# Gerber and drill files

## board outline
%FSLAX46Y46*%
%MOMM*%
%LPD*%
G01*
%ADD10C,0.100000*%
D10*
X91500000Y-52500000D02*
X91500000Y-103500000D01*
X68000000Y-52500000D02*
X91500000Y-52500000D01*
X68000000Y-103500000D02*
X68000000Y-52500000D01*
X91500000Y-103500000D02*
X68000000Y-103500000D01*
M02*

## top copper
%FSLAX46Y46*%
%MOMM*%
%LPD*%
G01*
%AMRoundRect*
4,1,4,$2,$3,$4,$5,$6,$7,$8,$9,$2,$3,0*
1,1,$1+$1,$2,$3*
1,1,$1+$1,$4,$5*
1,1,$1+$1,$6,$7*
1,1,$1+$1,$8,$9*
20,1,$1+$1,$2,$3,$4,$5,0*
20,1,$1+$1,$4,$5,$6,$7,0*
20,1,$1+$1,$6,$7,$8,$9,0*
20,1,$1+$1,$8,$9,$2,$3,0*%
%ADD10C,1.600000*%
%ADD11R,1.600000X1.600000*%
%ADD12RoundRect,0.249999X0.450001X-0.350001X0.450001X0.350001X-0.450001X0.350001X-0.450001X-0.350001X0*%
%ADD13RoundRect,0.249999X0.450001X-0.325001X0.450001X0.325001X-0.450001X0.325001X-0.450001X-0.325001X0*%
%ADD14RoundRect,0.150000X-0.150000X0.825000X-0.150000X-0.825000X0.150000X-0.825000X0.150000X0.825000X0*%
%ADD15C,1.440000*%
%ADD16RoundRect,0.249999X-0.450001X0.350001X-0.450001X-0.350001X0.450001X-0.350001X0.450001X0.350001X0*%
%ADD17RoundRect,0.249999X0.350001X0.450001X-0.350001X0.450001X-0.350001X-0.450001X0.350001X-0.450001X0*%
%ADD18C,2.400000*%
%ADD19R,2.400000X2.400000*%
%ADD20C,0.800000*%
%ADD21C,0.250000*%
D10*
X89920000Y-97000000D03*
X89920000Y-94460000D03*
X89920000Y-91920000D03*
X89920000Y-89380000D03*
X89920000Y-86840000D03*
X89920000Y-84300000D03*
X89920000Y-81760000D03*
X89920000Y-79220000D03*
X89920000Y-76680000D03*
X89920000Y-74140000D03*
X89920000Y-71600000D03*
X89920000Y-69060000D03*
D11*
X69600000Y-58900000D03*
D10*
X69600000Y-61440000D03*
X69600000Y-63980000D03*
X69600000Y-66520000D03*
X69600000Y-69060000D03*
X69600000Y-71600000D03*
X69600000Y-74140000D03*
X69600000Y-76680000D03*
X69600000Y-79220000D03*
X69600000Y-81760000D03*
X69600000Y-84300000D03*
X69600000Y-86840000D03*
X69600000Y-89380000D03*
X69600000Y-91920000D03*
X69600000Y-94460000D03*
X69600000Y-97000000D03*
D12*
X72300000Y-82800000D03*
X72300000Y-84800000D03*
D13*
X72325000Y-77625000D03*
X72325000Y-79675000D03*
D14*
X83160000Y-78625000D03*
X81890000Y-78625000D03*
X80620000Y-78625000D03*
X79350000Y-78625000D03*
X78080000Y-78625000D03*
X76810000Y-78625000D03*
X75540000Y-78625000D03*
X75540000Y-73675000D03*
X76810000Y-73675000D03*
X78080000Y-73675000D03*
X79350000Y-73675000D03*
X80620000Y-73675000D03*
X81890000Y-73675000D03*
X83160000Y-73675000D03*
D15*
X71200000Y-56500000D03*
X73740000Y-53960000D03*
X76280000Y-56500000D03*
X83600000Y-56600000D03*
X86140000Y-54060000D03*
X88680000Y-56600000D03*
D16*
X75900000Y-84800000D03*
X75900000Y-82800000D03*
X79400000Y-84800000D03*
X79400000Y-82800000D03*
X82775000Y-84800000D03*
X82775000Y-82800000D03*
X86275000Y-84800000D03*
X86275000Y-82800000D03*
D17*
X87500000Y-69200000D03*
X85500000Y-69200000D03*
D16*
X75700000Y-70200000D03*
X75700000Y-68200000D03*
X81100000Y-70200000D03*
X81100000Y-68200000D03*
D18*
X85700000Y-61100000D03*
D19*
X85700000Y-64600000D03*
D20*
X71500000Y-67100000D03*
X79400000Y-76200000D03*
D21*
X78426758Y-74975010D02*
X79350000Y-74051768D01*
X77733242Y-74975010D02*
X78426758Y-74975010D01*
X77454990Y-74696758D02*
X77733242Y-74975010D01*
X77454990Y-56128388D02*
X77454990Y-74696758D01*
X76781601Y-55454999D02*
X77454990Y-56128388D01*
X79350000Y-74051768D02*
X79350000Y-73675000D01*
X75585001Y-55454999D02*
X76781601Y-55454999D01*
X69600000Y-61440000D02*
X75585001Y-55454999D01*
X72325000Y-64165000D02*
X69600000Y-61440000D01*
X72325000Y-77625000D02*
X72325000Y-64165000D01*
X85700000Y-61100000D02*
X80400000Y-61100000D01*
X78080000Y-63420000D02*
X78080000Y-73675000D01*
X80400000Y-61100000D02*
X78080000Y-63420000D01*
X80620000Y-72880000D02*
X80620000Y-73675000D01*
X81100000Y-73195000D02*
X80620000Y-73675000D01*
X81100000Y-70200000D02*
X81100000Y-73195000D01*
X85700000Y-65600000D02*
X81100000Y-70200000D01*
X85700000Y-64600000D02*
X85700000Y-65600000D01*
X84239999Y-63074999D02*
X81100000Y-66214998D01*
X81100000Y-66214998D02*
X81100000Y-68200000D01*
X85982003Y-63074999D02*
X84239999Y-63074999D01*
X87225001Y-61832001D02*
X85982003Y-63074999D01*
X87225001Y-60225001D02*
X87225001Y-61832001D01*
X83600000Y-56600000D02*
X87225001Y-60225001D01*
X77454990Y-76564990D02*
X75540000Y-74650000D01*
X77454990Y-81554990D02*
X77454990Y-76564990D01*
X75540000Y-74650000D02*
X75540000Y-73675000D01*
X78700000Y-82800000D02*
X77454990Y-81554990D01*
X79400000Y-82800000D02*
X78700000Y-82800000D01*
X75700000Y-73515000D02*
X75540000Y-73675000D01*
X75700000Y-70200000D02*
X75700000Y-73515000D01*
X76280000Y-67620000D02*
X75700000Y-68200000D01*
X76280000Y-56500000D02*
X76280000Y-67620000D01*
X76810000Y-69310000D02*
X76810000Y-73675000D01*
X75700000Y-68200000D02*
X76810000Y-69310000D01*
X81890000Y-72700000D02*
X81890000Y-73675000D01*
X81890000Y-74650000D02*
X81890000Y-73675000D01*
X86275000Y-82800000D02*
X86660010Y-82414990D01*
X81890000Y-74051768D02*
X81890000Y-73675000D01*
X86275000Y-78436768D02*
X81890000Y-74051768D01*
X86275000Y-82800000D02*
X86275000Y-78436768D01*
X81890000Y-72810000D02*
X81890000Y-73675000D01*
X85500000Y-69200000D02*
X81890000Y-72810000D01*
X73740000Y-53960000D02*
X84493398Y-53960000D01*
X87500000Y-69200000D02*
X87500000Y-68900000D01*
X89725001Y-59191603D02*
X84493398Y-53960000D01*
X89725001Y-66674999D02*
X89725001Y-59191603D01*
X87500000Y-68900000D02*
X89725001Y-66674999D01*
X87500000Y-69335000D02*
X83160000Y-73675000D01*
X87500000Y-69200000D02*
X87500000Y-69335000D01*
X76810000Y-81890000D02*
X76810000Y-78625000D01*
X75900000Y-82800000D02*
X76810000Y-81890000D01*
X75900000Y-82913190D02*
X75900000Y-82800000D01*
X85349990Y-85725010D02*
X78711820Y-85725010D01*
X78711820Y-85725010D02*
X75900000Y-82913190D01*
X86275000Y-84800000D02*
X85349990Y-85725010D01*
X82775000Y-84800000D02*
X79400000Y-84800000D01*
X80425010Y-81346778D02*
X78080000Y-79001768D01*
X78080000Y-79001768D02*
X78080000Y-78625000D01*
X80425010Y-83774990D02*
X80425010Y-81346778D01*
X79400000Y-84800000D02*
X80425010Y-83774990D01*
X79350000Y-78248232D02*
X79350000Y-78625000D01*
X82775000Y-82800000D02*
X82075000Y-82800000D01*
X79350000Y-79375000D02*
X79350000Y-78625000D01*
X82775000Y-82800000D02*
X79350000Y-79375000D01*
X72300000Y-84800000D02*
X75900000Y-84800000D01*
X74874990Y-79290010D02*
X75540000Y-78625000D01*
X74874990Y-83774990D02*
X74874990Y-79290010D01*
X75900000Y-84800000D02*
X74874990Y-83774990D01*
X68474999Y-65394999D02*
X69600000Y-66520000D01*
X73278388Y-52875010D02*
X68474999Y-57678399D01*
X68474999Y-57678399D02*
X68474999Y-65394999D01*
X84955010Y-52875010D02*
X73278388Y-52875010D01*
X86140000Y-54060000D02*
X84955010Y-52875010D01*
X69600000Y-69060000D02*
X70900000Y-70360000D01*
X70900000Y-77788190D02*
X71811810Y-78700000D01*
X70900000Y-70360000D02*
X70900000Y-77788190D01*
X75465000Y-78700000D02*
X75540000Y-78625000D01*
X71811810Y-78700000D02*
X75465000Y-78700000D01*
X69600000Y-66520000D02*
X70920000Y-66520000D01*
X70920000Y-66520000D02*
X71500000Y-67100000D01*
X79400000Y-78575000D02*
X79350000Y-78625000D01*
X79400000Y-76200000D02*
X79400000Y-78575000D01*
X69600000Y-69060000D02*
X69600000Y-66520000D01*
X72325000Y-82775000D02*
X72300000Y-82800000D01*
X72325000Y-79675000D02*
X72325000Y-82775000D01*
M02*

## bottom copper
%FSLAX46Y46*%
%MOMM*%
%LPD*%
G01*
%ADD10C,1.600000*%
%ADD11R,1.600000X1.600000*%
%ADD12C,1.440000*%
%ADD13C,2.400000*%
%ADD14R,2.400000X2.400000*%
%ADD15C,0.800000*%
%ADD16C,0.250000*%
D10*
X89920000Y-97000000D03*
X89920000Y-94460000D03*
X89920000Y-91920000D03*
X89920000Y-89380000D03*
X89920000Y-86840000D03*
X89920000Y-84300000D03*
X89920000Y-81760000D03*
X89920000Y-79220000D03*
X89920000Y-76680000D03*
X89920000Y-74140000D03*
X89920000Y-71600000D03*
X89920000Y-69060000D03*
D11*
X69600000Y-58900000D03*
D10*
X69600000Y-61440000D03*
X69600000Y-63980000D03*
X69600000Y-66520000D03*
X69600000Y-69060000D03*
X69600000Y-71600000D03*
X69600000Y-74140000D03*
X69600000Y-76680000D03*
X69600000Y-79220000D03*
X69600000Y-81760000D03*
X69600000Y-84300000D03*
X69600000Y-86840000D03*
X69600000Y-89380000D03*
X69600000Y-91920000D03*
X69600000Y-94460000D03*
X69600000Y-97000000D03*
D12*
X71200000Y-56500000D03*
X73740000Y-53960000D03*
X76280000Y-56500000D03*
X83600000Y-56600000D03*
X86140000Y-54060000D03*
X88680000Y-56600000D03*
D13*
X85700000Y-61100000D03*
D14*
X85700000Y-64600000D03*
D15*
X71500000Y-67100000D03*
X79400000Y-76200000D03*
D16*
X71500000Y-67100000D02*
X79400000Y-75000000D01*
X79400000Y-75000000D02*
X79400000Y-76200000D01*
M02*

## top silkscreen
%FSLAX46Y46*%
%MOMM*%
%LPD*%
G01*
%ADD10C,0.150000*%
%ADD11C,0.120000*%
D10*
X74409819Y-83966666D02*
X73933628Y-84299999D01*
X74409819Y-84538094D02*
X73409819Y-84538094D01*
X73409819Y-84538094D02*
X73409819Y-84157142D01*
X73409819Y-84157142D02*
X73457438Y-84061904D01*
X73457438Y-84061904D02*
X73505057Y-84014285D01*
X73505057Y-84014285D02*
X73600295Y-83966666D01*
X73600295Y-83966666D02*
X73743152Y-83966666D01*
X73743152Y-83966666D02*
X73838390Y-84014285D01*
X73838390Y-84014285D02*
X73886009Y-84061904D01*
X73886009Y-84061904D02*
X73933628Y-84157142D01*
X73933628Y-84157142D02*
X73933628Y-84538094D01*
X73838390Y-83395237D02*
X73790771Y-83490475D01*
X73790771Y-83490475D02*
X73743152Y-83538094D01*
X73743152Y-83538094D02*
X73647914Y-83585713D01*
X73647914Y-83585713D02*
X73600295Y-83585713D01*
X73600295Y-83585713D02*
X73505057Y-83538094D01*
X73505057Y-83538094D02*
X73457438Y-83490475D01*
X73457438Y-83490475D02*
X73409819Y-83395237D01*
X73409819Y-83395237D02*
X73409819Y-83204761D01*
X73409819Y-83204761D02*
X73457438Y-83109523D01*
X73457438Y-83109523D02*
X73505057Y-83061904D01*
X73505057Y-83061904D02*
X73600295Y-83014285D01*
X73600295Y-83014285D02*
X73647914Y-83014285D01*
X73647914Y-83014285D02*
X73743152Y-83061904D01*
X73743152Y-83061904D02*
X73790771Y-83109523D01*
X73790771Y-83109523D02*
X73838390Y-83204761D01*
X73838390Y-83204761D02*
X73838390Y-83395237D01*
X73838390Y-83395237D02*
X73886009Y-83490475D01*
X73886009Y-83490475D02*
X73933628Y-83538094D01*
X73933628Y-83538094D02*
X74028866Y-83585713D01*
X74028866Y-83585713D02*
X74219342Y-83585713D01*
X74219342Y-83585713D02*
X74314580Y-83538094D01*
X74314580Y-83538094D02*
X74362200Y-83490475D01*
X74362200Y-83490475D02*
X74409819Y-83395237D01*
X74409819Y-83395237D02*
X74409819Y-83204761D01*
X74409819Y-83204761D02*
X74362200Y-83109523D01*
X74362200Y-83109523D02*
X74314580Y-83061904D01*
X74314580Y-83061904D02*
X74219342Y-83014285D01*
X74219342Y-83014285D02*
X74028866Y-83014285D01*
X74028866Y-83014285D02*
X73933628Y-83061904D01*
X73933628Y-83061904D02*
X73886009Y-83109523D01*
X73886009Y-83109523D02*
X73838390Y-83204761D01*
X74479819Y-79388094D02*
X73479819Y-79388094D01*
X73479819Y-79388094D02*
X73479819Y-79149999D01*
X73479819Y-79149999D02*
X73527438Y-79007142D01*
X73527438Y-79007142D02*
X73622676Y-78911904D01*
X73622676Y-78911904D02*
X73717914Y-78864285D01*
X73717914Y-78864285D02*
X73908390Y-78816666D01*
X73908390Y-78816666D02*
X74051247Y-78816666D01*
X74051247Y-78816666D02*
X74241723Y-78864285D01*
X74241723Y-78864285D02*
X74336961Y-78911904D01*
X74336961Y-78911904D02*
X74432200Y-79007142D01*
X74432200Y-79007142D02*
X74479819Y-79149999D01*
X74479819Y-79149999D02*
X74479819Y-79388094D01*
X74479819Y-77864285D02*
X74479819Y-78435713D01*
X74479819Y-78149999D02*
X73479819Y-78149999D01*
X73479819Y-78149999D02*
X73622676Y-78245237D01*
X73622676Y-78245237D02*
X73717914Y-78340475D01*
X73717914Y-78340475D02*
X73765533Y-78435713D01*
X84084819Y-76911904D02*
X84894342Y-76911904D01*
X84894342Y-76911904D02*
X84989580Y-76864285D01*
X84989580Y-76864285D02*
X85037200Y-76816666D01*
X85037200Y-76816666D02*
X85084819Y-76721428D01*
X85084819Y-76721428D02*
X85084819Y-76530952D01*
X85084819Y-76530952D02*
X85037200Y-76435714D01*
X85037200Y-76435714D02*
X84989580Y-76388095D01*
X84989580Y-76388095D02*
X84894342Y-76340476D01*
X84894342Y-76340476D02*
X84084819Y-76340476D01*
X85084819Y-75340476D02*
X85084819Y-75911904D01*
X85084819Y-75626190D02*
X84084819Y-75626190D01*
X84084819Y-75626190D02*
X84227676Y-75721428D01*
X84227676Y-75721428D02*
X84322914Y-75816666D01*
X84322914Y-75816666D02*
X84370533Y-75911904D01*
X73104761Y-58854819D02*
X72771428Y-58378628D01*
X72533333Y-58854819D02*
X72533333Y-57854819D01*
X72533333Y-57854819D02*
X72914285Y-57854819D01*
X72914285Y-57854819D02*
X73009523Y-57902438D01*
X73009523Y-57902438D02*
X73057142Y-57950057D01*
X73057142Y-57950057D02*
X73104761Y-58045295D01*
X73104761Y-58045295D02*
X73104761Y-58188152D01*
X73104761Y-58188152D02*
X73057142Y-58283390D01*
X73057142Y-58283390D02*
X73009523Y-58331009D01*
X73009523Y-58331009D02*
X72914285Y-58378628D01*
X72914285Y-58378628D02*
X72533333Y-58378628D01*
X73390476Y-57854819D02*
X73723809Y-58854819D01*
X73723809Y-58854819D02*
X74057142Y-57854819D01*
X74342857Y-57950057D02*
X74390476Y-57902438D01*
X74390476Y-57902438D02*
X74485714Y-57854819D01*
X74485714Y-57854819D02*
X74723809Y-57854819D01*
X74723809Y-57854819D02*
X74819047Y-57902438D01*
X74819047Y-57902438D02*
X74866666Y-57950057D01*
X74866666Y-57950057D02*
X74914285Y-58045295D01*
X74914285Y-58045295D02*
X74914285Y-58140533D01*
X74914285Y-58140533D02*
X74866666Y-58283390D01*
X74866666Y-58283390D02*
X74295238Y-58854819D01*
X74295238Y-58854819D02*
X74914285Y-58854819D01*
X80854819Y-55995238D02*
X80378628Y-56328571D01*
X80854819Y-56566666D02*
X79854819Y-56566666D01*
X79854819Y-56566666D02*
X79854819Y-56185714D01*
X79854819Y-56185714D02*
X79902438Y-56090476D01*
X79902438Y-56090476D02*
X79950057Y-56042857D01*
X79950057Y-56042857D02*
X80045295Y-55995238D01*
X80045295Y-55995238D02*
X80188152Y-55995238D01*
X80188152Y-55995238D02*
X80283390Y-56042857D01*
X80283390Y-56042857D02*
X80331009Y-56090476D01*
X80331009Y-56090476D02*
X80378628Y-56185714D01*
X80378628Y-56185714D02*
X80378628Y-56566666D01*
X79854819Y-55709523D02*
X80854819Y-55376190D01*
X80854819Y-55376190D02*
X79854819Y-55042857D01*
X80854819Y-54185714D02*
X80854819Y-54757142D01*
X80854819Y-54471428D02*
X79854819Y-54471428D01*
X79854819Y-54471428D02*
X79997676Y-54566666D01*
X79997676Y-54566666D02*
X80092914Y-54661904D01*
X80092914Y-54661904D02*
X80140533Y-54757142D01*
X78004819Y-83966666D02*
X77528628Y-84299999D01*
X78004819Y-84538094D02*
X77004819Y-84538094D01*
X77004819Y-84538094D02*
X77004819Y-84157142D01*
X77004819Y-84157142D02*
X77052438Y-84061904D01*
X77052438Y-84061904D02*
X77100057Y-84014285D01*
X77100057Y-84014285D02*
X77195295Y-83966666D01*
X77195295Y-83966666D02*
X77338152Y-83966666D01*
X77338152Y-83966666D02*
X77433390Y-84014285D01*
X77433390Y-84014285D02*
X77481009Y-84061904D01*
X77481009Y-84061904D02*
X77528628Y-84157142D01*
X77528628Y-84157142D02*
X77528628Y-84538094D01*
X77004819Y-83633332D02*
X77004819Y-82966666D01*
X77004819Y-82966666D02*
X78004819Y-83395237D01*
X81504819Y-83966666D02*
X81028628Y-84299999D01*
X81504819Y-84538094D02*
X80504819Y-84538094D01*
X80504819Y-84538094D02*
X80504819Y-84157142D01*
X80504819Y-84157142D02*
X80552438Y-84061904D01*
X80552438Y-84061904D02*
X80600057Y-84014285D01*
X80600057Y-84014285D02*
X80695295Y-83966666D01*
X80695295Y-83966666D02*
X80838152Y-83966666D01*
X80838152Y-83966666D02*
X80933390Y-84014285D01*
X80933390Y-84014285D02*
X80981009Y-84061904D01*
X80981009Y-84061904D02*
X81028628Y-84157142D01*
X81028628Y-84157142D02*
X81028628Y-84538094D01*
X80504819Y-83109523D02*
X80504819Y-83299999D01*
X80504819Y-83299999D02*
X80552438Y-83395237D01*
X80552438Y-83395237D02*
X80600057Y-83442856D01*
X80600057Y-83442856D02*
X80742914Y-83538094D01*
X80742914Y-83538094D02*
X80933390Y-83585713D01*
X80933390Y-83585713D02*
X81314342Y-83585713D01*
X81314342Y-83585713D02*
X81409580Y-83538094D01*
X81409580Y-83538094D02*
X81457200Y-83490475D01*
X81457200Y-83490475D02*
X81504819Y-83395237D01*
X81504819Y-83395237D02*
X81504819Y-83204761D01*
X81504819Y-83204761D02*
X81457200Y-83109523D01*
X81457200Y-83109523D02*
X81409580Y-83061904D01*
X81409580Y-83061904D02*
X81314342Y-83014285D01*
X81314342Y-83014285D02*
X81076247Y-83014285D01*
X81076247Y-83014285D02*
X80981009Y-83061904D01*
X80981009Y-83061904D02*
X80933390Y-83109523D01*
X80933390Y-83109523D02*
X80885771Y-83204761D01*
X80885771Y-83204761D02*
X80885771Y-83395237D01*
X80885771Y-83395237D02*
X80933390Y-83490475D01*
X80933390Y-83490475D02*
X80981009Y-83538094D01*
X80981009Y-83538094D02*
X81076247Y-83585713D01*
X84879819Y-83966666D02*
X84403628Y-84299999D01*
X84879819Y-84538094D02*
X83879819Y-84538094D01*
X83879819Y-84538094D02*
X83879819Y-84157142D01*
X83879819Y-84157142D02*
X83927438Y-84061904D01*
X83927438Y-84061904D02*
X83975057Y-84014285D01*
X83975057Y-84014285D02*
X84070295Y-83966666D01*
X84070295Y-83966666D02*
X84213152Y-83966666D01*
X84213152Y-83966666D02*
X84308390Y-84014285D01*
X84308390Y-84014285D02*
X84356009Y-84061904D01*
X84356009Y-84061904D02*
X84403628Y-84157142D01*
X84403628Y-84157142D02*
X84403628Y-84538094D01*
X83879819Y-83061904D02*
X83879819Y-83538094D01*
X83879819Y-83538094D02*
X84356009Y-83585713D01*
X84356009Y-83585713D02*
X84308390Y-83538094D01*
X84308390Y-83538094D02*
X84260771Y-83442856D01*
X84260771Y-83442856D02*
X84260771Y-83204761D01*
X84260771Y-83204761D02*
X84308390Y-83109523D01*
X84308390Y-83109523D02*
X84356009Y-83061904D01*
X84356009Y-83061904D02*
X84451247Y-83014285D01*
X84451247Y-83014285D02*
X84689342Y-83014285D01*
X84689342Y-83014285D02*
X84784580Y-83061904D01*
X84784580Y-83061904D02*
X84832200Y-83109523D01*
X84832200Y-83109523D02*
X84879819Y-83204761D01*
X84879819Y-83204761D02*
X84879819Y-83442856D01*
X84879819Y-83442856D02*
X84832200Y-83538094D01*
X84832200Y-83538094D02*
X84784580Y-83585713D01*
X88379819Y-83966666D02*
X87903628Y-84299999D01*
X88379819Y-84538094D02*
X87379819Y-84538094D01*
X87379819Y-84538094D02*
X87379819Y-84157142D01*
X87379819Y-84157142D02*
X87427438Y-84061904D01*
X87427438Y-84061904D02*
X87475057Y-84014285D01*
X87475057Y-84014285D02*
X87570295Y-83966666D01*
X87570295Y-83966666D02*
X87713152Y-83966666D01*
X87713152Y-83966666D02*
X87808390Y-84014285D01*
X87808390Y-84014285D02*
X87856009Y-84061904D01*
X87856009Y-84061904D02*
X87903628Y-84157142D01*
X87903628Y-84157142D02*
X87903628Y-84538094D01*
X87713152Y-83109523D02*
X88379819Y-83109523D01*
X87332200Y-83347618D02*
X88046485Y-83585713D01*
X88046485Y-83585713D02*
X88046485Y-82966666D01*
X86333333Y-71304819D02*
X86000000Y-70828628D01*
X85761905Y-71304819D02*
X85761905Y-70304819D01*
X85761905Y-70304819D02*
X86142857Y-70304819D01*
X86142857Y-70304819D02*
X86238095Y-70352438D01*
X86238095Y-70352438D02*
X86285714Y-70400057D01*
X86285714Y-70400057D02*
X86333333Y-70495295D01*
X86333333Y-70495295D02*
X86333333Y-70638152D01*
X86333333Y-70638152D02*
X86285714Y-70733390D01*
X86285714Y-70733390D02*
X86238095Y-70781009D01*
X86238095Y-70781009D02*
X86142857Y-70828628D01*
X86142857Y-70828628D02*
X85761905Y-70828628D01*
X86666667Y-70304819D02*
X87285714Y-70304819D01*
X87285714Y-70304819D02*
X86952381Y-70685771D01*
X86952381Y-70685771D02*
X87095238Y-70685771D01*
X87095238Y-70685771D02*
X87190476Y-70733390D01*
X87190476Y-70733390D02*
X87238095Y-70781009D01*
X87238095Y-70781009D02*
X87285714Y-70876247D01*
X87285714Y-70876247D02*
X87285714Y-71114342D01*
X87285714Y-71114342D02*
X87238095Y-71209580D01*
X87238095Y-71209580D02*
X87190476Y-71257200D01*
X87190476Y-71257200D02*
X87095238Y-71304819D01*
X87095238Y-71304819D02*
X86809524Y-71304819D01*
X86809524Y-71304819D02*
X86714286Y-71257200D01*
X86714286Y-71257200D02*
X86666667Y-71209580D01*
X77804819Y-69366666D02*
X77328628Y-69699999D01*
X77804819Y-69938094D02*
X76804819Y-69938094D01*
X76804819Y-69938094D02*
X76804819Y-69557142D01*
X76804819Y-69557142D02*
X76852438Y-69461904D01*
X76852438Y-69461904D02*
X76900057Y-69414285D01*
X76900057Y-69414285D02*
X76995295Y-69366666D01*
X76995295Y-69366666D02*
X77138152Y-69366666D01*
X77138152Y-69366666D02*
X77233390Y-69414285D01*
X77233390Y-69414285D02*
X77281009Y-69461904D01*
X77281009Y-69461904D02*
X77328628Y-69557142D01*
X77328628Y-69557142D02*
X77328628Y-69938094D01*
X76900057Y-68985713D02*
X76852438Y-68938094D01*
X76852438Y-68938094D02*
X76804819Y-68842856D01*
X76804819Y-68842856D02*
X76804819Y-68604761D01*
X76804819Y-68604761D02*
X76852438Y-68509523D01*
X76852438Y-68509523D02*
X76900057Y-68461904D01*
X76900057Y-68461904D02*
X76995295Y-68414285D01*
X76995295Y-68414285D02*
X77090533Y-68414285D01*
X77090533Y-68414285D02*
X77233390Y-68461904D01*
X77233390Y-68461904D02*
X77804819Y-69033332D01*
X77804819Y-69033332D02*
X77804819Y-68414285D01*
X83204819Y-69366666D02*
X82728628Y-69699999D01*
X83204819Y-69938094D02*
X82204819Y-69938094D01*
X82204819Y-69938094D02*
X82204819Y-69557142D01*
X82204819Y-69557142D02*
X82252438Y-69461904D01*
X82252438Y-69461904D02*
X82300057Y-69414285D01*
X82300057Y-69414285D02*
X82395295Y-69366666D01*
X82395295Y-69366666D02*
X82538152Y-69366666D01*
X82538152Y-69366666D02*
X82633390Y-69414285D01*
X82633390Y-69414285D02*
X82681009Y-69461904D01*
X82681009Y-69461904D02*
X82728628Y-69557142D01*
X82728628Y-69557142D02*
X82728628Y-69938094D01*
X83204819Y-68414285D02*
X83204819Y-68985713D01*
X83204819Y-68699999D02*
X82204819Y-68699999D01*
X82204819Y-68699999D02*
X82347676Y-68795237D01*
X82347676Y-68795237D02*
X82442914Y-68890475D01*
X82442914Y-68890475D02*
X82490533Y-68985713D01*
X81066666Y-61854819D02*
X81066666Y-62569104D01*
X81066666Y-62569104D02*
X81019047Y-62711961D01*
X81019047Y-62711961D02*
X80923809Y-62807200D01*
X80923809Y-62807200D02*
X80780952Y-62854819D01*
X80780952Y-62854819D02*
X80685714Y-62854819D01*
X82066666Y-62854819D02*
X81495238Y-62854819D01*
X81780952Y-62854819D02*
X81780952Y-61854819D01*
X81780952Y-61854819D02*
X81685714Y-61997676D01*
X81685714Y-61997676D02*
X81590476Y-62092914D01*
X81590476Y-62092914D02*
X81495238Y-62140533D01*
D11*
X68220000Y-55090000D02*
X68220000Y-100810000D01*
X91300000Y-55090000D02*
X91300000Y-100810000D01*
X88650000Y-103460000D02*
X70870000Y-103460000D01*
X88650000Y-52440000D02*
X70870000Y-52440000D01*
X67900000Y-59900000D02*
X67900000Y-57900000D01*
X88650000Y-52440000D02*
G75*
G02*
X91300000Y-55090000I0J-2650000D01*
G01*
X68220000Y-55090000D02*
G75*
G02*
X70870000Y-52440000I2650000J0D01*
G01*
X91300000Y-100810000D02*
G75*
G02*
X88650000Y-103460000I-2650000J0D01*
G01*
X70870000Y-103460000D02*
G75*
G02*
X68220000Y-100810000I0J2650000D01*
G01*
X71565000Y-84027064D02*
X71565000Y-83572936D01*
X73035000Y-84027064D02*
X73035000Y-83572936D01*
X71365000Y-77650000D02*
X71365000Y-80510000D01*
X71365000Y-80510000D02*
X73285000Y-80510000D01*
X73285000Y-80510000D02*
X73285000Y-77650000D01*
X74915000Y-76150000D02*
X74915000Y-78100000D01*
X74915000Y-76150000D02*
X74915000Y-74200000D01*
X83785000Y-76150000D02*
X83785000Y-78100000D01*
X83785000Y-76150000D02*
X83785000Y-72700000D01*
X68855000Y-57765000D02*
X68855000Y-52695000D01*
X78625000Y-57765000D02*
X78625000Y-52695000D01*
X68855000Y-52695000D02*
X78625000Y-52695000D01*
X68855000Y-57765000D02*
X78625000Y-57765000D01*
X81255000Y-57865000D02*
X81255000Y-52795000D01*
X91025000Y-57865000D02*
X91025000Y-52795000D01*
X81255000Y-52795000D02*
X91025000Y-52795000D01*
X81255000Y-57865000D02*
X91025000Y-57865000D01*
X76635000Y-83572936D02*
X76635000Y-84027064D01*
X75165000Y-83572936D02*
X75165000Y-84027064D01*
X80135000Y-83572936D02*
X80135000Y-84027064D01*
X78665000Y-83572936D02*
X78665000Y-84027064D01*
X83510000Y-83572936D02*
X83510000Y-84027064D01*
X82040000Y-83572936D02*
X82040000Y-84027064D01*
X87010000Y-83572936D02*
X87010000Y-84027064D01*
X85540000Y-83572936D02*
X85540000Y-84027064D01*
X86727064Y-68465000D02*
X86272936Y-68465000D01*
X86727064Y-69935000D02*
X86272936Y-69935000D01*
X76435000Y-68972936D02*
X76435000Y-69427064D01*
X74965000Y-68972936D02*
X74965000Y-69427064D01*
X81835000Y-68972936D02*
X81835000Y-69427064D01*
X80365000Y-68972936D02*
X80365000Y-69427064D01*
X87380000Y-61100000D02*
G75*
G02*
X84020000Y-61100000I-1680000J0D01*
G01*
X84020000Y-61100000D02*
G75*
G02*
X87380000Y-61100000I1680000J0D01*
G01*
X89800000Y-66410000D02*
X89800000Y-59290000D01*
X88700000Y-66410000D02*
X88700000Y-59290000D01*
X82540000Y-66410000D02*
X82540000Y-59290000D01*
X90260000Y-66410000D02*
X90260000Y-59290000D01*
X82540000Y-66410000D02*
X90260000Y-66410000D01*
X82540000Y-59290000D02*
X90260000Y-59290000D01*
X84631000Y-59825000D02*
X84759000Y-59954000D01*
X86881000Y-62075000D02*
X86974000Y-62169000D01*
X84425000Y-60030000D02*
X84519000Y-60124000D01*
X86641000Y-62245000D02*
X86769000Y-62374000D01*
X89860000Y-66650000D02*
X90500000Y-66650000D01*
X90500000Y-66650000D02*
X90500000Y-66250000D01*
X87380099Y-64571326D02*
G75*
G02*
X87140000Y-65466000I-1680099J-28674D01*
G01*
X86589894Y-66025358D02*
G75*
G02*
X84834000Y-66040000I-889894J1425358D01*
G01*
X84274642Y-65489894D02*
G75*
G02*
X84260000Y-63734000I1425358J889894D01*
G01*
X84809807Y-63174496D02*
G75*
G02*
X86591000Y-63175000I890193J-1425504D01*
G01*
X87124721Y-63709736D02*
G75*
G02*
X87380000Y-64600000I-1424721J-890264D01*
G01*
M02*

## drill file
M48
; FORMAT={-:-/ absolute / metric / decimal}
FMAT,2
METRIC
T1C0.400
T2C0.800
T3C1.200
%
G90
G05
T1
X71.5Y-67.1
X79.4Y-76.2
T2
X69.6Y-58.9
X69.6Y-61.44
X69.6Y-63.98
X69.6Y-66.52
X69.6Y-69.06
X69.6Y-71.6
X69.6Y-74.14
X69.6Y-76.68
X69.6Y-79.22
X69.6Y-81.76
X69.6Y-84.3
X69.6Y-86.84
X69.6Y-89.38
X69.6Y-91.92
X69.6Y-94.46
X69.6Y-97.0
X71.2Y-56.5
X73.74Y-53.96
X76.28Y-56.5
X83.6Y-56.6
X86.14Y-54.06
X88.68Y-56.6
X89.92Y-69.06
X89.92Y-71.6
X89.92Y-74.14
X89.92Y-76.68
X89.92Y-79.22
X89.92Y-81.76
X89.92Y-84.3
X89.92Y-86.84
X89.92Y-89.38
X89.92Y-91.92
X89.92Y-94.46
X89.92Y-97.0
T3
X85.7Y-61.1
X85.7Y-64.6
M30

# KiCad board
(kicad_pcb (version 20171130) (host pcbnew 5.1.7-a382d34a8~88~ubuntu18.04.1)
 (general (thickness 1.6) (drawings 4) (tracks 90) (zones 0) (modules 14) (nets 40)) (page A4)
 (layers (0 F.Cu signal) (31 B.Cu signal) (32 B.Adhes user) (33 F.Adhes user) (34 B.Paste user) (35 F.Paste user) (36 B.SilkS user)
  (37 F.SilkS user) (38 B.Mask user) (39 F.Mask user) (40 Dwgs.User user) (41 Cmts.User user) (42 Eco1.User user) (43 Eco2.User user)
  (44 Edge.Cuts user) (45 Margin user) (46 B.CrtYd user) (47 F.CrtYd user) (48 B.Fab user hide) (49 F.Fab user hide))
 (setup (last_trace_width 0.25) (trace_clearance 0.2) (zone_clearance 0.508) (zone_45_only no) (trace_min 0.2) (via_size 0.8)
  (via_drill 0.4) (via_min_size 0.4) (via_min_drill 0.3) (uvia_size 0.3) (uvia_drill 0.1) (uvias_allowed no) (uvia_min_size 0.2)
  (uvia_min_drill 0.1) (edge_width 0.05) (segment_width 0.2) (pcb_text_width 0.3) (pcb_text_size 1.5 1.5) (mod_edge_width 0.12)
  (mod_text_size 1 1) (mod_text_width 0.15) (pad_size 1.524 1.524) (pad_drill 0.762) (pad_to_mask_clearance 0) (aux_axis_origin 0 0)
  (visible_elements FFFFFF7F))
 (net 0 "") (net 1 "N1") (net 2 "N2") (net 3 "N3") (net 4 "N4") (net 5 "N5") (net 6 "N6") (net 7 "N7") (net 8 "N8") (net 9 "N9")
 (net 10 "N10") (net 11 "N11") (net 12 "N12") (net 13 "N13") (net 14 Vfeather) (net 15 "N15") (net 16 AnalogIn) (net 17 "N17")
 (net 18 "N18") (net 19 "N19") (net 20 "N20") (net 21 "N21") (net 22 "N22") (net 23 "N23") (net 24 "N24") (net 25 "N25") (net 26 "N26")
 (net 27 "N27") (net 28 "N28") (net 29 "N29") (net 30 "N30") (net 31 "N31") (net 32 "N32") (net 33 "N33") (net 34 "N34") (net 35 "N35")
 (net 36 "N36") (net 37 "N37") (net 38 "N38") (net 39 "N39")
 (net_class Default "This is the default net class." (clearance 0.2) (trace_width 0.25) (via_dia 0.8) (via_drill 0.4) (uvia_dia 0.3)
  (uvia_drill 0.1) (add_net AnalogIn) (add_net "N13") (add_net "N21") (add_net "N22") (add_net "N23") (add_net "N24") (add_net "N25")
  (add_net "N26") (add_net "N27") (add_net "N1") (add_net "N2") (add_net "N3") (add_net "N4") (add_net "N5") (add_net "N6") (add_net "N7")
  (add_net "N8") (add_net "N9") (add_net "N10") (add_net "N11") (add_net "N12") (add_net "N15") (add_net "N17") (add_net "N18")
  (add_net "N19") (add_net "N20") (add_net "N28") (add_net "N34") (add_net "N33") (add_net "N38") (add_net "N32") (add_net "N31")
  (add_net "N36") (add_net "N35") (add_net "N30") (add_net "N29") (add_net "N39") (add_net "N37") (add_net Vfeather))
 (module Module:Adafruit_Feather (layer F.Cu) (at 69.6 58.9)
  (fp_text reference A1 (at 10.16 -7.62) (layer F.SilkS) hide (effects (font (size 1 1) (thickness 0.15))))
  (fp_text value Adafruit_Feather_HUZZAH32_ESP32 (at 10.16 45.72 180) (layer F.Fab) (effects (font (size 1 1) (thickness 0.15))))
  (fp_line (start -1.38 -3.81) (end -1.38 41.91) (layer F.SilkS) (width 0.12))
  (fp_line (start 21.7 -3.81) (end 21.7 41.91) (layer F.SilkS) (width 0.12))
  (fp_line (start 19.05 44.56) (end 1.27 44.56) (layer F.SilkS) (width 0.12))
  (fp_line (start 19.05 -6.46) (end 1.27 -6.46) (layer F.SilkS) (width 0.12))
  (fp_line (start -1.7 1) (end -1.7 -1) (layer F.SilkS) (width 0.12))
  (fp_arc (start 19.05 -3.81) (end 21.7 -3.81) (angle -90) (layer F.SilkS) (width 0.12))
  (fp_arc (start 1.27 -3.81) (end 1.27 -6.46) (angle -90) (layer F.SilkS) (width 0.12))
  (fp_arc (start 19.05 41.91) (end 19.05 44.56) (angle -90) (layer F.SilkS) (width 0.12))
  (fp_arc (start 1.27 41.91) (end -1.38 41.91) (angle -90) (layer F.SilkS) (width 0.12))
  (pad 17 thru_hole circle (at 20.32 38.1 180) (size 1.6 1.6) (drill 0.8) (layers *.Cu *.Mask) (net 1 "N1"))
  (pad 18 thru_hole circle (at 20.32 35.56 180) (size 1.6 1.6) (drill 0.8) (layers *.Cu *.Mask) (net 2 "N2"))
  (pad 19 thru_hole circle (at 20.32 33.02 180) (size 1.6 1.6) (drill 0.8) (layers *.Cu *.Mask) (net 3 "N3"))
  (pad 20 thru_hole circle (at 20.32 30.48 180) (size 1.6 1.6) (drill 0.8) (layers *.Cu *.Mask) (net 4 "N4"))
  (pad 21 thru_hole circle (at 20.32 27.94 180) (size 1.6 1.6) (drill 0.8) (layers *.Cu *.Mask) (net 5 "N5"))
  (pad 22 thru_hole circle (at 20.32 25.4 180) (size 1.6 1.6) (drill 0.8) (layers *.Cu *.Mask) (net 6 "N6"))
  (pad 23 thru_hole circle (at 20.32 22.86 180) (size 1.6 1.6) (drill 0.8) (layers *.Cu *.Mask) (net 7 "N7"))
  (pad 24 thru_hole circle (at 20.32 20.32 180) (size 1.6 1.6) (drill 0.8) (layers *.Cu *.Mask) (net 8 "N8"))
  (pad 25 thru_hole circle (at 20.32 17.78 180) (size 1.6 1.6) (drill 0.8) (layers *.Cu *.Mask) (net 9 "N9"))
  (pad 26 thru_hole circle (at 20.32 15.24 180) (size 1.6 1.6) (drill 0.8) (layers *.Cu *.Mask) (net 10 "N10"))
  (pad 27 thru_hole circle (at 20.32 12.7 180) (size 1.6 1.6) (drill 0.8) (layers *.Cu *.Mask) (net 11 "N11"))
  (pad 28 thru_hole circle (at 20.32 10.16 180) (size 1.6 1.6) (drill 0.8) (layers *.Cu *.Mask) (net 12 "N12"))
  (pad 1 thru_hole rect (at 0 0 180) (size 1.6 1.6) (drill 0.8) (layers *.Cu *.Mask) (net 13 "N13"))
  (pad 2 thru_hole circle (at 0 2.54 180) (size 1.6 1.6) (drill 0.8) (layers *.Cu *.Mask) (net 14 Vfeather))
  (pad 3 thru_hole circle (at 0 5.08 180) (size 1.6 1.6) (drill 0.8) (layers *.Cu *.Mask) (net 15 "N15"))
  (pad 4 thru_hole circle (at 0 7.62 180) (size 1.6 1.6) (drill 0.8) (layers *.Cu *.Mask) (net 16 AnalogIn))
  (pad 5 thru_hole circle (at 0 10.16 180) (size 1.6 1.6) (drill 0.8) (layers *.Cu *.Mask) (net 16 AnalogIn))
  (pad 6 thru_hole circle (at 0 12.7 180) (size 1.6 1.6) (drill 0.8) (layers *.Cu *.Mask) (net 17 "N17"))
  (pad 7 thru_hole circle (at 0 15.24 180) (size 1.6 1.6) (drill 0.8) (layers *.Cu *.Mask) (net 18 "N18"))
  (pad 8 thru_hole circle (at 0 17.78 180) (size 1.6 1.6) (drill 0.8) (layers *.Cu *.Mask) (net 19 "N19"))
  (pad 9 thru_hole circle (at 0 20.32 180) (size 1.6 1.6) (drill 0.8) (layers *.Cu *.Mask) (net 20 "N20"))
  (pad 10 thru_hole circle (at 0 22.86 180) (size 1.6 1.6) (drill 0.8) (layers *.Cu *.Mask) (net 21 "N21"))
  (pad 11 thru_hole circle (at 0 25.4 180) (size 1.6 1.6) (drill 0.8) (layers *.Cu *.Mask) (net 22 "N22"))
  (pad 12 thru_hole circle (at 0 27.94 180) (size 1.6 1.6) (drill 0.8) (layers *.Cu *.Mask) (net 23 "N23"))
  (pad 13 thru_hole circle (at 0 30.48 180) (size 1.6 1.6) (drill 0.8) (layers *.Cu *.Mask) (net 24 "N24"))
  (pad 14 thru_hole circle (at 0 33.02 180) (size 1.6 1.6) (drill 0.8) (layers *.Cu *.Mask) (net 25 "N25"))
  (pad 15 thru_hole circle (at 0 35.56 180) (size 1.6 1.6) (drill 0.8) (layers *.Cu *.Mask) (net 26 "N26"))
  (pad 16 thru_hole circle (at 0 38.1 180) (size 1.6 1.6) (drill 0.8) (layers *.Cu *.Mask) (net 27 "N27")))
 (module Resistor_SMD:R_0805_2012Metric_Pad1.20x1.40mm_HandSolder (layer F.Cu) (at 72.3 83.8 90)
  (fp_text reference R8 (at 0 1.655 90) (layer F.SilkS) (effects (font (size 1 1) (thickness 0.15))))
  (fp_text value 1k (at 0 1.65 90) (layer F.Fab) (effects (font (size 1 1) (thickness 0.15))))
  (fp_line (start -0.227064 -0.735) (end 0.227064 -0.735) (layer F.SilkS) (width 0.12))
  (fp_line (start -0.227064 0.735) (end 0.227064 0.735) (layer F.SilkS) (width 0.12))
  (pad 2 smd roundrect (at 1 0 90) (size 1.2 1.4) (layers F.Cu F.Paste F.Mask) (roundrect_rratio 0.2083325) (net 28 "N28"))
  (pad 1 smd roundrect (at -1 0 90) (size 1.2 1.4) (layers F.Cu F.Paste F.Mask) (roundrect_rratio 0.2083325) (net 16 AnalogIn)))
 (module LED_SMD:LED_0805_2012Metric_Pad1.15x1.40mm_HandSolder (layer F.Cu) (at 72.325 78.65 90)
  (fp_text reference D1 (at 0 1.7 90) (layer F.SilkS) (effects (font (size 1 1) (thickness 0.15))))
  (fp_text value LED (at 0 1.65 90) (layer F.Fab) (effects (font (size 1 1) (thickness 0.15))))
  (fp_line (start 1 -0.96) (end -1.86 -0.96) (layer F.SilkS) (width 0.12))
  (fp_line (start -1.86 -0.96) (end -1.86 0.96) (layer F.SilkS) (width 0.12))
  (fp_line (start -1.86 0.96) (end 1 0.96) (layer F.SilkS) (width 0.12))
  (pad 2 smd roundrect (at 1.025 0 90) (size 1.15 1.4) (layers F.Cu F.Paste F.Mask) (roundrect_rratio 0.2173904347826087) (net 14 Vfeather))
  (pad 1 smd roundrect (at -1.025 0 90) (size 1.15 1.4) (layers F.Cu F.Paste F.Mask) (roundrect_rratio 0.2173904347826087) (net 28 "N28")))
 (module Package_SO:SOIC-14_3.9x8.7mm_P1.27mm (layer F.Cu) (at 79.35 76.15 270)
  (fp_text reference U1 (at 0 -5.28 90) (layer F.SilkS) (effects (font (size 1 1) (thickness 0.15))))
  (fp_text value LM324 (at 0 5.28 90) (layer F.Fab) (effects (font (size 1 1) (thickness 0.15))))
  (fp_line (start 0 4.435) (end 1.95 4.435) (layer F.SilkS) (width 0.12))
  (fp_line (start 0 4.435) (end -1.95 4.435) (layer F.SilkS) (width 0.12))
  (fp_line (start 0 -4.435) (end 1.95 -4.435) (layer F.SilkS) (width 0.12))
  (fp_line (start 0 -4.435) (end -3.45 -4.435) (layer F.SilkS) (width 0.12))
  (pad 14 smd roundrect (at 2.475 -3.81 270) (size 1.95 0.6) (layers F.Cu F.Paste F.Mask) (roundrect_rratio 0.25))
  (pad 13 smd roundrect (at 2.475 -2.54 270) (size 1.95 0.6) (layers F.Cu F.Paste F.Mask) (roundrect_rratio 0.25))
  (pad 12 smd roundrect (at 2.475 -1.27 270) (size 1.95 0.6) (layers F.Cu F.Paste F.Mask) (roundrect_rratio 0.25))
  (pad 11 smd roundrect (at 2.475 0 270) (size 1.95 0.6) (layers F.Cu F.Paste F.Mask) (roundrect_rratio 0.25) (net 16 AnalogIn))
  (pad 10 smd roundrect (at 2.475 1.27 270) (size 1.95 0.6) (layers F.Cu F.Paste F.Mask) (roundrect_rratio 0.25) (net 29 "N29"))
  (pad 9 smd roundrect (at 2.475 2.54 270) (size 1.95 0.6) (layers F.Cu F.Paste F.Mask) (roundrect_rratio 0.25) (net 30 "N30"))
  (pad 8 smd roundrect (at 2.475 3.81 270) (size 1.95 0.6) (layers F.Cu F.Paste F.Mask) (roundrect_rratio 0.25) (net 16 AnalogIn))
  (pad 7 smd roundrect (at -2.475 3.81 270) (size 1.95 0.6) (layers F.Cu F.Paste F.Mask) (roundrect_rratio 0.25) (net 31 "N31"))
  (pad 6 smd roundrect (at -2.475 2.54 270) (size 1.95 0.6) (layers F.Cu F.Paste F.Mask) (roundrect_rratio 0.25) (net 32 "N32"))
  (pad 5 smd roundrect (at -2.475 1.27 270) (size 1.95 0.6) (layers F.Cu F.Paste F.Mask) (roundrect_rratio 0.25) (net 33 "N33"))
  (pad 4 smd roundrect (at -2.475 0 270) (size 1.95 0.6) (layers F.Cu F.Paste F.Mask) (roundrect_rratio 0.25) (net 14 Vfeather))
  (pad 3 smd roundrect (at -2.475 -1.27 270) (size 1.95 0.6) (layers F.Cu F.Paste F.Mask) (roundrect_rratio 0.25) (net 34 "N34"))
  (pad 2 smd roundrect (at -2.475 -2.54 270) (size 1.95 0.6) (layers F.Cu F.Paste F.Mask) (roundrect_rratio 0.25) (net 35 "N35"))
  (pad 1 smd roundrect (at -2.475 -3.81 270) (size 1.95 0.6) (layers F.Cu F.Paste F.Mask) (roundrect_rratio 0.25) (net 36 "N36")))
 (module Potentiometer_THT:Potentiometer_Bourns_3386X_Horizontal (layer F.Cu) (at 71.2 56.5 90)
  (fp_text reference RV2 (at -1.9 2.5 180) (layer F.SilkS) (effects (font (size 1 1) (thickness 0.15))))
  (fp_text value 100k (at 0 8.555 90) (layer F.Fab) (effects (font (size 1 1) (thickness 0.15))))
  (fp_line (start -1.265 -2.345) (end 3.805 -2.345) (layer F.SilkS) (width 0.12))
  (fp_line (start -1.265 7.425) (end 3.805 7.425) (layer F.SilkS) (width 0.12))
  (fp_line (start 3.805 -2.345) (end 3.805 7.425) (layer F.SilkS) (width 0.12))
  (fp_line (start -1.265 -2.345) (end -1.265 7.425) (layer F.SilkS) (width 0.12))
  (pad 1 thru_hole circle (at 0 0 90) (size 1.44 1.44) (drill 0.8) (layers *.Cu *.Mask) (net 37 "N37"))
  (pad 2 thru_hole circle (at 2.54 2.54 90) (size 1.44 1.44) (drill 0.8) (layers *.Cu *.Mask) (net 36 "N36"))
  (pad 3 thru_hole circle (at 0 5.08 90) (size 1.44 1.44) (drill 0.8) (layers *.Cu *.Mask) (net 32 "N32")))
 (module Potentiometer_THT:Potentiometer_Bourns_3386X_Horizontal (layer F.Cu) (at 83.6 56.6 90)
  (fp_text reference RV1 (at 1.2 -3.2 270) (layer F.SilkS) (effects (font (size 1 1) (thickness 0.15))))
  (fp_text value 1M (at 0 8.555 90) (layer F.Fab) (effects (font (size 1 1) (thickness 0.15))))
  (fp_line (start -1.265 -2.345) (end 3.805 -2.345) (layer F.SilkS) (width 0.12))
  (fp_line (start -1.265 7.425) (end 3.805 7.425) (layer F.SilkS) (width 0.12))
  (fp_line (start 3.805 -2.345) (end 3.805 7.425) (layer F.SilkS) (width 0.12))
  (fp_line (start -1.265 -2.345) (end -1.265 7.425) (layer F.SilkS) (width 0.12))
  (pad 1 thru_hole circle (at 0 0 90) (size 1.44 1.44) (drill 0.8) (layers *.Cu *.Mask) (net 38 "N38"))
  (pad 2 thru_hole circle (at 2.54 2.54 90) (size 1.44 1.44) (drill 0.8) (layers *.Cu *.Mask) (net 16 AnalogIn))
  (pad 3 thru_hole circle (at 0 5.08 90) (size 1.44 1.44) (drill 0.8) (layers *.Cu *.Mask) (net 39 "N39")))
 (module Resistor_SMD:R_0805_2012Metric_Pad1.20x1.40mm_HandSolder (layer F.Cu) (at 75.9 83.8 270)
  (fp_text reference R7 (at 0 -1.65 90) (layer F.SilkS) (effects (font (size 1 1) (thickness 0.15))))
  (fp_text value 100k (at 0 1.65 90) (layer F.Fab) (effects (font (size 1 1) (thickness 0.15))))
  (fp_line (start -0.227064 -0.735) (end 0.227064 -0.735) (layer F.SilkS) (width 0.12))
  (fp_line (start -0.227064 0.735) (end 0.227064 0.735) (layer F.SilkS) (width 0.12))
  (pad 2 smd roundrect (at 1 0 270) (size 1.2 1.4) (layers F.Cu F.Paste F.Mask) (roundrect_rratio 0.2083325) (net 16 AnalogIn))
  (pad 1 smd roundrect (at -1 0 270) (size 1.2 1.4) (layers F.Cu F.Paste F.Mask) (roundrect_rratio 0.2083325) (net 30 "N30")))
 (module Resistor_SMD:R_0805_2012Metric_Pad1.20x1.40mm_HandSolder (layer F.Cu) (at 79.4 83.8 270)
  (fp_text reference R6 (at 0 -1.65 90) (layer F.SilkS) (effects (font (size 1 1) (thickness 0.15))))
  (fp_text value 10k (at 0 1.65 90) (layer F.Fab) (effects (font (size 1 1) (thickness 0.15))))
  (fp_line (start -0.227064 -0.735) (end 0.227064 -0.735) (layer F.SilkS) (width 0.12))
  (fp_line (start -0.227064 0.735) (end 0.227064 0.735) (layer F.SilkS) (width 0.12))
  (pad 2 smd roundrect (at 1 0 270) (size 1.2 1.4) (layers F.Cu F.Paste F.Mask) (roundrect_rratio 0.2083325) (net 29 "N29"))
  (pad 1 smd roundrect (at -1 0 270) (size 1.2 1.4) (layers F.Cu F.Paste F.Mask) (roundrect_rratio 0.2083325) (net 31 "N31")))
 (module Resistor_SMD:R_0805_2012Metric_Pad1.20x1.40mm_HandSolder (layer F.Cu) (at 82.775 83.8 270)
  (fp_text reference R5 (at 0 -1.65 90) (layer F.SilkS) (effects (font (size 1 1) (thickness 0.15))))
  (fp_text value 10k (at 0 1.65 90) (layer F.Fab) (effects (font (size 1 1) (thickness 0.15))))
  (fp_line (start -0.227064 -0.735) (end 0.227064 -0.735) (layer F.SilkS) (width 0.12))
  (fp_line (start -0.227064 0.735) (end 0.227064 0.735) (layer F.SilkS) (width 0.12))
  (pad 2 smd roundrect (at 1 0 270) (size 1.2 1.4) (layers F.Cu F.Paste F.Mask) (roundrect_rratio 0.2083325) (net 29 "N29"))
  (pad 1 smd roundrect (at -1 0 270) (size 1.2 1.4) (layers F.Cu F.Paste F.Mask) (roundrect_rratio 0.2083325) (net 16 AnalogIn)))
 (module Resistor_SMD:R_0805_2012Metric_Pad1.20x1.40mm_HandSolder (layer F.Cu) (at 86.275 83.8 270)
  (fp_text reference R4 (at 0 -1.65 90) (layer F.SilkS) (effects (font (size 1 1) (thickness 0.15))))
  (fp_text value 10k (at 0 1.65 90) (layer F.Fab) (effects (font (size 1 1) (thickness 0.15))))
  (fp_line (start -0.227064 -0.735) (end 0.227064 -0.735) (layer F.SilkS) (width 0.12))
  (fp_line (start -0.227064 0.735) (end 0.227064 0.735) (layer F.SilkS) (width 0.12))
  (pad 2 smd roundrect (at 1 0 270) (size 1.2 1.4) (layers F.Cu F.Paste F.Mask) (roundrect_rratio 0.2083325) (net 30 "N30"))
  (pad 1 smd roundrect (at -1 0 270) (size 1.2 1.4) (layers F.Cu F.Paste F.Mask) (roundrect_rratio 0.2083325) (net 35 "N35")))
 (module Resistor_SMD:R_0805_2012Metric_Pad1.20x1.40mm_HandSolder (layer F.Cu) (at 86.5 69.2 180)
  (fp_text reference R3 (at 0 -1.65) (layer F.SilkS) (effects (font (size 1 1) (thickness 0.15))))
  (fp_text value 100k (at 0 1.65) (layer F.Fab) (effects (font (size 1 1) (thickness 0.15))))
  (fp_line (start -0.227064 0.735) (end 0.227064 0.735) (layer F.SilkS) (width 0.12))
  (fp_line (start -0.227064 -0.735) (end 0.227064 -0.735) (layer F.SilkS) (width 0.12))
  (pad 1 smd roundrect (at -1 0 180) (size 1.2 1.4) (layers F.Cu F.Paste F.Mask) (roundrect_rratio 0.2083325) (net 36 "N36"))
  (pad 2 smd roundrect (at 1 0 180) (size 1.2 1.4) (layers F.Cu F.Paste F.Mask) (roundrect_rratio 0.2083325) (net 35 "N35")))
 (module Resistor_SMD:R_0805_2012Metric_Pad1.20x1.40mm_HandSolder (layer F.Cu) (at 75.7 69.2 270)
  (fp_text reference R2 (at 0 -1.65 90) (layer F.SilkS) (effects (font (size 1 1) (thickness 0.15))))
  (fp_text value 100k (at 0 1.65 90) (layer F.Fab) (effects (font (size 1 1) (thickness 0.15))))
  (fp_line (start -0.227064 -0.735) (end 0.227064 -0.735) (layer F.SilkS) (width 0.12))
  (fp_line (start -0.227064 0.735) (end 0.227064 0.735) (layer F.SilkS) (width 0.12))
  (pad 2 smd roundrect (at 1 0 270) (size 1.2 1.4) (layers F.Cu F.Paste F.Mask) (roundrect_rratio 0.2083325) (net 31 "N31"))
  (pad 1 smd roundrect (at -1 0 270) (size 1.2 1.4) (layers F.Cu F.Paste F.Mask) (roundrect_rratio 0.2083325) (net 32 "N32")))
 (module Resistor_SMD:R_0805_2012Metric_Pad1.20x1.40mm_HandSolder (layer F.Cu) (at 81.1 69.2 270)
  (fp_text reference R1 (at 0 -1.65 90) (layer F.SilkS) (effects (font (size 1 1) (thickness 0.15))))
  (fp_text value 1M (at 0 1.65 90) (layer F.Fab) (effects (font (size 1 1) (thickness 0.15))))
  (fp_line (start -0.227064 -0.735) (end 0.227064 -0.735) (layer F.SilkS) (width 0.12))
  (fp_line (start -0.227064 0.735) (end 0.227064 0.735) (layer F.SilkS) (width 0.12))
  (pad 2 smd roundrect (at 1 0 270) (size 1.2 1.4) (layers F.Cu F.Paste F.Mask) (roundrect_rratio 0.2083325) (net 34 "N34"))
  (pad 1 smd roundrect (at -1 0 270) (size 1.2 1.4) (layers F.Cu F.Paste F.Mask) (roundrect_rratio 0.2083325) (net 38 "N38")))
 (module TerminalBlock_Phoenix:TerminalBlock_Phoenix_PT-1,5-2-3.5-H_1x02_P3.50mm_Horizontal (layer F.Cu) (at 85.7 64.6 90)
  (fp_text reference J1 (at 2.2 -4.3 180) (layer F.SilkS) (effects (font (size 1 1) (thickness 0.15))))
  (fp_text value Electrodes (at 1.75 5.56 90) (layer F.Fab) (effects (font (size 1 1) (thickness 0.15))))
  (fp_circle (center 3.5 0) (end 5.18 0) (layer F.SilkS) (width 0.12))
  (fp_line (start -1.81 4.1) (end 5.31 4.1) (layer F.SilkS) (width 0.12))
  (fp_line (start -1.81 3) (end 5.31 3) (layer F.SilkS) (width 0.12))
  (fp_line (start -1.81 -3.16) (end 5.31 -3.16) (layer F.SilkS) (width 0.12))
  (fp_line (start -1.81 4.56) (end 5.31 4.56) (layer F.SilkS) (width 0.12))
  (fp_line (start -1.81 -3.16) (end -1.81 4.56) (layer F.SilkS) (width 0.12))
  (fp_line (start 5.31 -3.16) (end 5.31 4.56) (layer F.SilkS) (width 0.12))
  (fp_line (start 4.775 -1.069) (end 4.646 -0.941) (layer F.SilkS) (width 0.12))
  (fp_line (start 2.525 1.181) (end 2.431 1.274) (layer F.SilkS) (width 0.12))
  (fp_line (start 4.57 -1.275) (end 4.476 -1.181) (layer F.SilkS) (width 0.12))
  (fp_line (start 2.355 0.941) (end 2.226 1.069) (layer F.SilkS) (width 0.12))
  (fp_line (start -2.05 4.16) (end -2.05 4.8) (layer F.SilkS) (width 0.12))
  (fp_line (start -2.05 4.8) (end -1.65 4.8) (layer F.SilkS) (width 0.12))
  (fp_arc (start 0 0) (end -0.866 1.44) (angle -32) (layer F.SilkS) (width 0.12))
  (fp_arc (start 0 0) (end -1.44 -0.866) (angle -63) (layer F.SilkS) (width 0.12))
  (fp_arc (start 0 0) (end 0.866 -1.44) (angle -63) (layer F.SilkS) (width 0.12))
  (fp_arc (start 0 0) (end 1.425 0.891) (angle -64) (layer F.SilkS) (width 0.12))
  (fp_arc (start 0 0) (end 0 1.68) (angle -32) (layer F.SilkS) (width 0.12))
  (pad 2 thru_hole circle (at 3.5 0 90) (size 2.4 2.4) (drill 1.2) (layers *.Cu *.Mask) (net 33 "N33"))
  (pad 1 thru_hole rect (at 0 0 90) (size 2.4 2.4) (drill 1.2) (layers *.Cu *.Mask) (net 34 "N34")))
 (gr_line (start 91.5 52.5) (end 91.5 103.5) (layer Edge.Cuts) (width 0.1))
 (gr_line (start 68 52.5) (end 91.5 52.5) (layer Edge.Cuts) (width 0.1))
 (gr_line (start 68 103.5) (end 68 52.5) (layer Edge.Cuts) (width 0.1))
 (gr_line (start 91.5 103.5) (end 68 103.5) (layer Edge.Cuts) (width 0.1))
 (segment (start 78.426758 74.97501) (end 79.35 74.051768) (width 0.25) (layer F.Cu) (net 14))
 (segment (start 77.733242 74.97501) (end 78.426758 74.97501) (width 0.25) (layer F.Cu) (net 14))
 (segment (start 77.45499 74.696758) (end 77.733242 74.97501) (width 0.25) (layer F.Cu) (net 14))
 (segment (start 77.45499 56.128388) (end 77.45499 74.696758) (width 0.25) (layer F.Cu) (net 14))
 (segment (start 76.781601 55.454999) (end 77.45499 56.128388) (width 0.25) (layer F.Cu) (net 14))
 (segment (start 79.35 74.051768) (end 79.35 73.675) (width 0.25) (layer F.Cu) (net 14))
 (segment (start 75.585001 55.454999) (end 76.781601 55.454999) (width 0.25) (layer F.Cu) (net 14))
 (segment (start 69.6 61.44) (end 75.585001 55.454999) (width 0.25) (layer F.Cu) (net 14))
 (segment (start 72.325 64.165) (end 69.6 61.44) (width 0.25) (layer F.Cu) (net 14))
 (segment (start 72.325 77.625) (end 72.325 64.165) (width 0.25) (layer F.Cu) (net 14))
 (segment (start 85.7 61.1) (end 80.4 61.1) (width 0.25) (layer F.Cu) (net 33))
 (segment (start 78.08 63.42) (end 78.08 73.675) (width 0.25) (layer F.Cu) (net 33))
 (segment (start 80.4 61.1) (end 78.08 63.42) (width 0.25) (layer F.Cu) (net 33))
 (segment (start 80.62 72.88) (end 80.62 73.675) (width 0.25) (layer F.Cu) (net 34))
 (segment (start 81.1 73.195) (end 80.62 73.675) (width 0.25) (layer F.Cu) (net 34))
 (segment (start 81.1 70.2) (end 81.1 73.195) (width 0.25) (layer F.Cu) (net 34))
 (segment (start 85.7 65.6) (end 81.1 70.2) (width 0.25) (layer F.Cu) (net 34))
 (segment (start 85.7 64.6) (end 85.7 65.6) (width 0.25) (layer F.Cu) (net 34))
 (segment (start 84.239999 63.074999) (end 81.1 66.214998) (width 0.25) (layer F.Cu) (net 38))
 (segment (start 81.1 66.214998) (end 81.1 68.2) (width 0.25) (layer F.Cu) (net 38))
 (segment (start 85.982003 63.074999) (end 84.239999 63.074999) (width 0.25) (layer F.Cu) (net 38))
 (segment (start 87.225001 61.832001) (end 85.982003 63.074999) (width 0.25) (layer F.Cu) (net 38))
 (segment (start 87.225001 60.225001) (end 87.225001 61.832001) (width 0.25) (layer F.Cu) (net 38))
 (segment (start 83.6 56.6) (end 87.225001 60.225001) (width 0.25) (layer F.Cu) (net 38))
 (segment (start 77.45499 76.56499) (end 75.54 74.65) (width 0.25) (layer F.Cu) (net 31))
 (segment (start 77.45499 81.55499) (end 77.45499 76.56499) (width 0.25) (layer F.Cu) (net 31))
 (segment (start 75.54 74.65) (end 75.54 73.675) (width 0.25) (layer F.Cu) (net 31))
 (segment (start 78.7 82.8) (end 77.45499 81.55499) (width 0.25) (layer F.Cu) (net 31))
 (segment (start 79.4 82.8) (end 78.7 82.8) (width 0.25) (layer F.Cu) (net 31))
 (segment (start 75.7 73.515) (end 75.54 73.675) (width 0.25) (layer F.Cu) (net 31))
 (segment (start 75.7 70.2) (end 75.7 73.515) (width 0.25) (layer F.Cu) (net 31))
 (segment (start 76.28 67.62) (end 75.7 68.2) (width 0.25) (layer F.Cu) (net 32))
 (segment (start 76.28 56.5) (end 76.28 67.62) (width 0.25) (layer F.Cu) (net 32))
 (segment (start 76.81 69.31) (end 76.81 73.675) (width 0.25) (layer F.Cu) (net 32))
 (segment (start 75.7 68.2) (end 76.81 69.31) (width 0.25) (layer F.Cu) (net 32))
 (segment (start 81.89 72.7) (end 81.89 73.675) (width 0.25) (layer F.Cu) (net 35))
 (segment (start 81.89 74.65) (end 81.89 73.675) (width 0.25) (layer F.Cu) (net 35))
 (segment (start 86.275 82.8) (end 86.66001 82.41499) (width 0.25) (layer F.Cu) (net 35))
 (segment (start 81.89 74.051768) (end 81.89 73.675) (width 0.25) (layer F.Cu) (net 35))
 (segment (start 86.275 78.436768) (end 81.89 74.051768) (width 0.25) (layer F.Cu) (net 35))
 (segment (start 86.275 82.8) (end 86.275 78.436768) (width 0.25) (layer F.Cu) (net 35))
 (segment (start 81.89 72.81) (end 81.89 73.675) (width 0.25) (layer F.Cu) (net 35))
 (segment (start 85.5 69.2) (end 81.89 72.81) (width 0.25) (layer F.Cu) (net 35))
 (segment (start 73.74 53.96) (end 84.493398 53.96) (width 0.25) (layer F.Cu) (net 36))
 (segment (start 87.5 69.2) (end 87.5 68.9) (width 0.25) (layer F.Cu) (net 36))
 (segment (start 89.725001 59.191603) (end 84.493398 53.96) (width 0.25) (layer F.Cu) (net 36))
 (segment (start 89.725001 66.674999) (end 89.725001 59.191603) (width 0.25) (layer F.Cu) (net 36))
 (segment (start 87.5 68.9) (end 89.725001 66.674999) (width 0.25) (layer F.Cu) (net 36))
 (segment (start 87.5 69.335) (end 83.16 73.675) (width 0.25) (layer F.Cu) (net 36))
 (segment (start 87.5 69.2) (end 87.5 69.335) (width 0.25) (layer F.Cu) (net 36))
 (segment (start 76.81 81.89) (end 76.81 78.625) (width 0.25) (layer F.Cu) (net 30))
 (segment (start 75.9 82.8) (end 76.81 81.89) (width 0.25) (layer F.Cu) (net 30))
 (segment (start 75.9 82.91319) (end 75.9 82.8) (width 0.25) (layer F.Cu) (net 30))
 (segment (start 85.34999 85.72501) (end 78.71182 85.72501) (width 0.25) (layer F.Cu) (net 30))
 (segment (start 78.71182 85.72501) (end 75.9 82.91319) (width 0.25) (layer F.Cu) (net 30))
 (segment (start 86.275 84.8) (end 85.34999 85.72501) (width 0.25) (layer F.Cu) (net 30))
 (segment (start 82.775 84.8) (end 79.4 84.8) (width 0.25) (layer F.Cu) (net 29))
 (segment (start 80.42501 81.346778) (end 78.08 79.001768) (width 0.25) (layer F.Cu) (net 29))
 (segment (start 78.08 79.001768) (end 78.08 78.625) (width 0.25) (layer F.Cu) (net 29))
 (segment (start 80.42501 83.77499) (end 80.42501 81.346778) (width 0.25) (layer F.Cu) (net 29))
 (segment (start 79.4 84.8) (end 80.42501 83.77499) (width 0.25) (layer F.Cu) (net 29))
 (segment (start 79.35 78.248232) (end 79.35 78.625) (width 0.25) (layer F.Cu) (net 16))
 (segment (start 82.775 82.8) (end 82.075 82.8) (width 0.25) (layer F.Cu) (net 16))
 (segment (start 79.35 79.375) (end 79.35 78.625) (width 0.25) (layer F.Cu) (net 16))
 (segment (start 82.775 82.8) (end 79.35 79.375) (width 0.25) (layer F.Cu) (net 16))
 (segment (start 72.3 84.8) (end 75.9 84.8) (width 0.25) (layer F.Cu) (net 16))
 (segment (start 74.87499 79.29001) (end 75.54 78.625) (width 0.25) (layer F.Cu) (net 16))
 (segment (start 74.87499 83.77499) (end 74.87499 79.29001) (width 0.25) (layer F.Cu) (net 16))
 (segment (start 75.9 84.8) (end 74.87499 83.77499) (width 0.25) (layer F.Cu) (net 16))
 (segment (start 68.474999 65.394999) (end 69.6 66.52) (width 0.25) (layer F.Cu) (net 16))
 (segment (start 73.278388 52.87501) (end 68.474999 57.678399) (width 0.25) (layer F.Cu) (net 16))
 (segment (start 68.474999 57.678399) (end 68.474999 65.394999) (width 0.25) (layer F.Cu) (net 16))
 (segment (start 84.95501 52.87501) (end 73.278388 52.87501) (width 0.25) (layer F.Cu) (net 16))
 (segment (start 86.14 54.06) (end 84.95501 52.87501) (width 0.25) (layer F.Cu) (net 16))
 (segment (start 69.6 69.06) (end 70.9 70.36) (width 0.25) (layer F.Cu) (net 16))
 (segment (start 70.9 77.78819) (end 71.81181 78.7) (width 0.25) (layer F.Cu) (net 16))
 (segment (start 70.9 70.36) (end 70.9 77.78819) (width 0.25) (layer F.Cu) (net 16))
 (segment (start 75.465 78.7) (end 75.54 78.625) (width 0.25) (layer F.Cu) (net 16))
 (segment (start 71.81181 78.7) (end 75.465 78.7) (width 0.25) (layer F.Cu) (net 16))
 (via (at 71.5 67.1) (size 0.8) (drill 0.4) (layers F.Cu B.Cu) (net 16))
 (segment (start 69.6 66.52) (end 70.92 66.52) (width 0.25) (layer F.Cu) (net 16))
 (segment (start 70.92 66.52) (end 71.5 67.1) (width 0.25) (layer F.Cu) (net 16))
 (via (at 79.4 76.2) (size 0.8) (drill 0.4) (layers F.Cu B.Cu) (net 16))
 (segment (start 71.5 67.1) (end 79.4 75) (width 0.25) (layer B.Cu) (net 16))
 (segment (start 79.4 75) (end 79.4 76.2) (width 0.25) (layer B.Cu) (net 16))
 (segment (start 79.4 78.575) (end 79.35 78.625) (width 0.25) (layer F.Cu) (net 16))
 (segment (start 79.4 76.2) (end 79.4 78.575) (width 0.25) (layer F.Cu) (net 16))
 (segment (start 69.6 69.06) (end 69.6 66.52) (width 0.25) (layer F.Cu) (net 16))
 (segment (start 72.325 82.775) (end 72.3 82.8) (width 0.25) (layer F.Cu) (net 28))
 (segment (start 72.325 79.675) (end 72.325 82.775) (width 0.25) (layer F.Cu) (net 28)))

